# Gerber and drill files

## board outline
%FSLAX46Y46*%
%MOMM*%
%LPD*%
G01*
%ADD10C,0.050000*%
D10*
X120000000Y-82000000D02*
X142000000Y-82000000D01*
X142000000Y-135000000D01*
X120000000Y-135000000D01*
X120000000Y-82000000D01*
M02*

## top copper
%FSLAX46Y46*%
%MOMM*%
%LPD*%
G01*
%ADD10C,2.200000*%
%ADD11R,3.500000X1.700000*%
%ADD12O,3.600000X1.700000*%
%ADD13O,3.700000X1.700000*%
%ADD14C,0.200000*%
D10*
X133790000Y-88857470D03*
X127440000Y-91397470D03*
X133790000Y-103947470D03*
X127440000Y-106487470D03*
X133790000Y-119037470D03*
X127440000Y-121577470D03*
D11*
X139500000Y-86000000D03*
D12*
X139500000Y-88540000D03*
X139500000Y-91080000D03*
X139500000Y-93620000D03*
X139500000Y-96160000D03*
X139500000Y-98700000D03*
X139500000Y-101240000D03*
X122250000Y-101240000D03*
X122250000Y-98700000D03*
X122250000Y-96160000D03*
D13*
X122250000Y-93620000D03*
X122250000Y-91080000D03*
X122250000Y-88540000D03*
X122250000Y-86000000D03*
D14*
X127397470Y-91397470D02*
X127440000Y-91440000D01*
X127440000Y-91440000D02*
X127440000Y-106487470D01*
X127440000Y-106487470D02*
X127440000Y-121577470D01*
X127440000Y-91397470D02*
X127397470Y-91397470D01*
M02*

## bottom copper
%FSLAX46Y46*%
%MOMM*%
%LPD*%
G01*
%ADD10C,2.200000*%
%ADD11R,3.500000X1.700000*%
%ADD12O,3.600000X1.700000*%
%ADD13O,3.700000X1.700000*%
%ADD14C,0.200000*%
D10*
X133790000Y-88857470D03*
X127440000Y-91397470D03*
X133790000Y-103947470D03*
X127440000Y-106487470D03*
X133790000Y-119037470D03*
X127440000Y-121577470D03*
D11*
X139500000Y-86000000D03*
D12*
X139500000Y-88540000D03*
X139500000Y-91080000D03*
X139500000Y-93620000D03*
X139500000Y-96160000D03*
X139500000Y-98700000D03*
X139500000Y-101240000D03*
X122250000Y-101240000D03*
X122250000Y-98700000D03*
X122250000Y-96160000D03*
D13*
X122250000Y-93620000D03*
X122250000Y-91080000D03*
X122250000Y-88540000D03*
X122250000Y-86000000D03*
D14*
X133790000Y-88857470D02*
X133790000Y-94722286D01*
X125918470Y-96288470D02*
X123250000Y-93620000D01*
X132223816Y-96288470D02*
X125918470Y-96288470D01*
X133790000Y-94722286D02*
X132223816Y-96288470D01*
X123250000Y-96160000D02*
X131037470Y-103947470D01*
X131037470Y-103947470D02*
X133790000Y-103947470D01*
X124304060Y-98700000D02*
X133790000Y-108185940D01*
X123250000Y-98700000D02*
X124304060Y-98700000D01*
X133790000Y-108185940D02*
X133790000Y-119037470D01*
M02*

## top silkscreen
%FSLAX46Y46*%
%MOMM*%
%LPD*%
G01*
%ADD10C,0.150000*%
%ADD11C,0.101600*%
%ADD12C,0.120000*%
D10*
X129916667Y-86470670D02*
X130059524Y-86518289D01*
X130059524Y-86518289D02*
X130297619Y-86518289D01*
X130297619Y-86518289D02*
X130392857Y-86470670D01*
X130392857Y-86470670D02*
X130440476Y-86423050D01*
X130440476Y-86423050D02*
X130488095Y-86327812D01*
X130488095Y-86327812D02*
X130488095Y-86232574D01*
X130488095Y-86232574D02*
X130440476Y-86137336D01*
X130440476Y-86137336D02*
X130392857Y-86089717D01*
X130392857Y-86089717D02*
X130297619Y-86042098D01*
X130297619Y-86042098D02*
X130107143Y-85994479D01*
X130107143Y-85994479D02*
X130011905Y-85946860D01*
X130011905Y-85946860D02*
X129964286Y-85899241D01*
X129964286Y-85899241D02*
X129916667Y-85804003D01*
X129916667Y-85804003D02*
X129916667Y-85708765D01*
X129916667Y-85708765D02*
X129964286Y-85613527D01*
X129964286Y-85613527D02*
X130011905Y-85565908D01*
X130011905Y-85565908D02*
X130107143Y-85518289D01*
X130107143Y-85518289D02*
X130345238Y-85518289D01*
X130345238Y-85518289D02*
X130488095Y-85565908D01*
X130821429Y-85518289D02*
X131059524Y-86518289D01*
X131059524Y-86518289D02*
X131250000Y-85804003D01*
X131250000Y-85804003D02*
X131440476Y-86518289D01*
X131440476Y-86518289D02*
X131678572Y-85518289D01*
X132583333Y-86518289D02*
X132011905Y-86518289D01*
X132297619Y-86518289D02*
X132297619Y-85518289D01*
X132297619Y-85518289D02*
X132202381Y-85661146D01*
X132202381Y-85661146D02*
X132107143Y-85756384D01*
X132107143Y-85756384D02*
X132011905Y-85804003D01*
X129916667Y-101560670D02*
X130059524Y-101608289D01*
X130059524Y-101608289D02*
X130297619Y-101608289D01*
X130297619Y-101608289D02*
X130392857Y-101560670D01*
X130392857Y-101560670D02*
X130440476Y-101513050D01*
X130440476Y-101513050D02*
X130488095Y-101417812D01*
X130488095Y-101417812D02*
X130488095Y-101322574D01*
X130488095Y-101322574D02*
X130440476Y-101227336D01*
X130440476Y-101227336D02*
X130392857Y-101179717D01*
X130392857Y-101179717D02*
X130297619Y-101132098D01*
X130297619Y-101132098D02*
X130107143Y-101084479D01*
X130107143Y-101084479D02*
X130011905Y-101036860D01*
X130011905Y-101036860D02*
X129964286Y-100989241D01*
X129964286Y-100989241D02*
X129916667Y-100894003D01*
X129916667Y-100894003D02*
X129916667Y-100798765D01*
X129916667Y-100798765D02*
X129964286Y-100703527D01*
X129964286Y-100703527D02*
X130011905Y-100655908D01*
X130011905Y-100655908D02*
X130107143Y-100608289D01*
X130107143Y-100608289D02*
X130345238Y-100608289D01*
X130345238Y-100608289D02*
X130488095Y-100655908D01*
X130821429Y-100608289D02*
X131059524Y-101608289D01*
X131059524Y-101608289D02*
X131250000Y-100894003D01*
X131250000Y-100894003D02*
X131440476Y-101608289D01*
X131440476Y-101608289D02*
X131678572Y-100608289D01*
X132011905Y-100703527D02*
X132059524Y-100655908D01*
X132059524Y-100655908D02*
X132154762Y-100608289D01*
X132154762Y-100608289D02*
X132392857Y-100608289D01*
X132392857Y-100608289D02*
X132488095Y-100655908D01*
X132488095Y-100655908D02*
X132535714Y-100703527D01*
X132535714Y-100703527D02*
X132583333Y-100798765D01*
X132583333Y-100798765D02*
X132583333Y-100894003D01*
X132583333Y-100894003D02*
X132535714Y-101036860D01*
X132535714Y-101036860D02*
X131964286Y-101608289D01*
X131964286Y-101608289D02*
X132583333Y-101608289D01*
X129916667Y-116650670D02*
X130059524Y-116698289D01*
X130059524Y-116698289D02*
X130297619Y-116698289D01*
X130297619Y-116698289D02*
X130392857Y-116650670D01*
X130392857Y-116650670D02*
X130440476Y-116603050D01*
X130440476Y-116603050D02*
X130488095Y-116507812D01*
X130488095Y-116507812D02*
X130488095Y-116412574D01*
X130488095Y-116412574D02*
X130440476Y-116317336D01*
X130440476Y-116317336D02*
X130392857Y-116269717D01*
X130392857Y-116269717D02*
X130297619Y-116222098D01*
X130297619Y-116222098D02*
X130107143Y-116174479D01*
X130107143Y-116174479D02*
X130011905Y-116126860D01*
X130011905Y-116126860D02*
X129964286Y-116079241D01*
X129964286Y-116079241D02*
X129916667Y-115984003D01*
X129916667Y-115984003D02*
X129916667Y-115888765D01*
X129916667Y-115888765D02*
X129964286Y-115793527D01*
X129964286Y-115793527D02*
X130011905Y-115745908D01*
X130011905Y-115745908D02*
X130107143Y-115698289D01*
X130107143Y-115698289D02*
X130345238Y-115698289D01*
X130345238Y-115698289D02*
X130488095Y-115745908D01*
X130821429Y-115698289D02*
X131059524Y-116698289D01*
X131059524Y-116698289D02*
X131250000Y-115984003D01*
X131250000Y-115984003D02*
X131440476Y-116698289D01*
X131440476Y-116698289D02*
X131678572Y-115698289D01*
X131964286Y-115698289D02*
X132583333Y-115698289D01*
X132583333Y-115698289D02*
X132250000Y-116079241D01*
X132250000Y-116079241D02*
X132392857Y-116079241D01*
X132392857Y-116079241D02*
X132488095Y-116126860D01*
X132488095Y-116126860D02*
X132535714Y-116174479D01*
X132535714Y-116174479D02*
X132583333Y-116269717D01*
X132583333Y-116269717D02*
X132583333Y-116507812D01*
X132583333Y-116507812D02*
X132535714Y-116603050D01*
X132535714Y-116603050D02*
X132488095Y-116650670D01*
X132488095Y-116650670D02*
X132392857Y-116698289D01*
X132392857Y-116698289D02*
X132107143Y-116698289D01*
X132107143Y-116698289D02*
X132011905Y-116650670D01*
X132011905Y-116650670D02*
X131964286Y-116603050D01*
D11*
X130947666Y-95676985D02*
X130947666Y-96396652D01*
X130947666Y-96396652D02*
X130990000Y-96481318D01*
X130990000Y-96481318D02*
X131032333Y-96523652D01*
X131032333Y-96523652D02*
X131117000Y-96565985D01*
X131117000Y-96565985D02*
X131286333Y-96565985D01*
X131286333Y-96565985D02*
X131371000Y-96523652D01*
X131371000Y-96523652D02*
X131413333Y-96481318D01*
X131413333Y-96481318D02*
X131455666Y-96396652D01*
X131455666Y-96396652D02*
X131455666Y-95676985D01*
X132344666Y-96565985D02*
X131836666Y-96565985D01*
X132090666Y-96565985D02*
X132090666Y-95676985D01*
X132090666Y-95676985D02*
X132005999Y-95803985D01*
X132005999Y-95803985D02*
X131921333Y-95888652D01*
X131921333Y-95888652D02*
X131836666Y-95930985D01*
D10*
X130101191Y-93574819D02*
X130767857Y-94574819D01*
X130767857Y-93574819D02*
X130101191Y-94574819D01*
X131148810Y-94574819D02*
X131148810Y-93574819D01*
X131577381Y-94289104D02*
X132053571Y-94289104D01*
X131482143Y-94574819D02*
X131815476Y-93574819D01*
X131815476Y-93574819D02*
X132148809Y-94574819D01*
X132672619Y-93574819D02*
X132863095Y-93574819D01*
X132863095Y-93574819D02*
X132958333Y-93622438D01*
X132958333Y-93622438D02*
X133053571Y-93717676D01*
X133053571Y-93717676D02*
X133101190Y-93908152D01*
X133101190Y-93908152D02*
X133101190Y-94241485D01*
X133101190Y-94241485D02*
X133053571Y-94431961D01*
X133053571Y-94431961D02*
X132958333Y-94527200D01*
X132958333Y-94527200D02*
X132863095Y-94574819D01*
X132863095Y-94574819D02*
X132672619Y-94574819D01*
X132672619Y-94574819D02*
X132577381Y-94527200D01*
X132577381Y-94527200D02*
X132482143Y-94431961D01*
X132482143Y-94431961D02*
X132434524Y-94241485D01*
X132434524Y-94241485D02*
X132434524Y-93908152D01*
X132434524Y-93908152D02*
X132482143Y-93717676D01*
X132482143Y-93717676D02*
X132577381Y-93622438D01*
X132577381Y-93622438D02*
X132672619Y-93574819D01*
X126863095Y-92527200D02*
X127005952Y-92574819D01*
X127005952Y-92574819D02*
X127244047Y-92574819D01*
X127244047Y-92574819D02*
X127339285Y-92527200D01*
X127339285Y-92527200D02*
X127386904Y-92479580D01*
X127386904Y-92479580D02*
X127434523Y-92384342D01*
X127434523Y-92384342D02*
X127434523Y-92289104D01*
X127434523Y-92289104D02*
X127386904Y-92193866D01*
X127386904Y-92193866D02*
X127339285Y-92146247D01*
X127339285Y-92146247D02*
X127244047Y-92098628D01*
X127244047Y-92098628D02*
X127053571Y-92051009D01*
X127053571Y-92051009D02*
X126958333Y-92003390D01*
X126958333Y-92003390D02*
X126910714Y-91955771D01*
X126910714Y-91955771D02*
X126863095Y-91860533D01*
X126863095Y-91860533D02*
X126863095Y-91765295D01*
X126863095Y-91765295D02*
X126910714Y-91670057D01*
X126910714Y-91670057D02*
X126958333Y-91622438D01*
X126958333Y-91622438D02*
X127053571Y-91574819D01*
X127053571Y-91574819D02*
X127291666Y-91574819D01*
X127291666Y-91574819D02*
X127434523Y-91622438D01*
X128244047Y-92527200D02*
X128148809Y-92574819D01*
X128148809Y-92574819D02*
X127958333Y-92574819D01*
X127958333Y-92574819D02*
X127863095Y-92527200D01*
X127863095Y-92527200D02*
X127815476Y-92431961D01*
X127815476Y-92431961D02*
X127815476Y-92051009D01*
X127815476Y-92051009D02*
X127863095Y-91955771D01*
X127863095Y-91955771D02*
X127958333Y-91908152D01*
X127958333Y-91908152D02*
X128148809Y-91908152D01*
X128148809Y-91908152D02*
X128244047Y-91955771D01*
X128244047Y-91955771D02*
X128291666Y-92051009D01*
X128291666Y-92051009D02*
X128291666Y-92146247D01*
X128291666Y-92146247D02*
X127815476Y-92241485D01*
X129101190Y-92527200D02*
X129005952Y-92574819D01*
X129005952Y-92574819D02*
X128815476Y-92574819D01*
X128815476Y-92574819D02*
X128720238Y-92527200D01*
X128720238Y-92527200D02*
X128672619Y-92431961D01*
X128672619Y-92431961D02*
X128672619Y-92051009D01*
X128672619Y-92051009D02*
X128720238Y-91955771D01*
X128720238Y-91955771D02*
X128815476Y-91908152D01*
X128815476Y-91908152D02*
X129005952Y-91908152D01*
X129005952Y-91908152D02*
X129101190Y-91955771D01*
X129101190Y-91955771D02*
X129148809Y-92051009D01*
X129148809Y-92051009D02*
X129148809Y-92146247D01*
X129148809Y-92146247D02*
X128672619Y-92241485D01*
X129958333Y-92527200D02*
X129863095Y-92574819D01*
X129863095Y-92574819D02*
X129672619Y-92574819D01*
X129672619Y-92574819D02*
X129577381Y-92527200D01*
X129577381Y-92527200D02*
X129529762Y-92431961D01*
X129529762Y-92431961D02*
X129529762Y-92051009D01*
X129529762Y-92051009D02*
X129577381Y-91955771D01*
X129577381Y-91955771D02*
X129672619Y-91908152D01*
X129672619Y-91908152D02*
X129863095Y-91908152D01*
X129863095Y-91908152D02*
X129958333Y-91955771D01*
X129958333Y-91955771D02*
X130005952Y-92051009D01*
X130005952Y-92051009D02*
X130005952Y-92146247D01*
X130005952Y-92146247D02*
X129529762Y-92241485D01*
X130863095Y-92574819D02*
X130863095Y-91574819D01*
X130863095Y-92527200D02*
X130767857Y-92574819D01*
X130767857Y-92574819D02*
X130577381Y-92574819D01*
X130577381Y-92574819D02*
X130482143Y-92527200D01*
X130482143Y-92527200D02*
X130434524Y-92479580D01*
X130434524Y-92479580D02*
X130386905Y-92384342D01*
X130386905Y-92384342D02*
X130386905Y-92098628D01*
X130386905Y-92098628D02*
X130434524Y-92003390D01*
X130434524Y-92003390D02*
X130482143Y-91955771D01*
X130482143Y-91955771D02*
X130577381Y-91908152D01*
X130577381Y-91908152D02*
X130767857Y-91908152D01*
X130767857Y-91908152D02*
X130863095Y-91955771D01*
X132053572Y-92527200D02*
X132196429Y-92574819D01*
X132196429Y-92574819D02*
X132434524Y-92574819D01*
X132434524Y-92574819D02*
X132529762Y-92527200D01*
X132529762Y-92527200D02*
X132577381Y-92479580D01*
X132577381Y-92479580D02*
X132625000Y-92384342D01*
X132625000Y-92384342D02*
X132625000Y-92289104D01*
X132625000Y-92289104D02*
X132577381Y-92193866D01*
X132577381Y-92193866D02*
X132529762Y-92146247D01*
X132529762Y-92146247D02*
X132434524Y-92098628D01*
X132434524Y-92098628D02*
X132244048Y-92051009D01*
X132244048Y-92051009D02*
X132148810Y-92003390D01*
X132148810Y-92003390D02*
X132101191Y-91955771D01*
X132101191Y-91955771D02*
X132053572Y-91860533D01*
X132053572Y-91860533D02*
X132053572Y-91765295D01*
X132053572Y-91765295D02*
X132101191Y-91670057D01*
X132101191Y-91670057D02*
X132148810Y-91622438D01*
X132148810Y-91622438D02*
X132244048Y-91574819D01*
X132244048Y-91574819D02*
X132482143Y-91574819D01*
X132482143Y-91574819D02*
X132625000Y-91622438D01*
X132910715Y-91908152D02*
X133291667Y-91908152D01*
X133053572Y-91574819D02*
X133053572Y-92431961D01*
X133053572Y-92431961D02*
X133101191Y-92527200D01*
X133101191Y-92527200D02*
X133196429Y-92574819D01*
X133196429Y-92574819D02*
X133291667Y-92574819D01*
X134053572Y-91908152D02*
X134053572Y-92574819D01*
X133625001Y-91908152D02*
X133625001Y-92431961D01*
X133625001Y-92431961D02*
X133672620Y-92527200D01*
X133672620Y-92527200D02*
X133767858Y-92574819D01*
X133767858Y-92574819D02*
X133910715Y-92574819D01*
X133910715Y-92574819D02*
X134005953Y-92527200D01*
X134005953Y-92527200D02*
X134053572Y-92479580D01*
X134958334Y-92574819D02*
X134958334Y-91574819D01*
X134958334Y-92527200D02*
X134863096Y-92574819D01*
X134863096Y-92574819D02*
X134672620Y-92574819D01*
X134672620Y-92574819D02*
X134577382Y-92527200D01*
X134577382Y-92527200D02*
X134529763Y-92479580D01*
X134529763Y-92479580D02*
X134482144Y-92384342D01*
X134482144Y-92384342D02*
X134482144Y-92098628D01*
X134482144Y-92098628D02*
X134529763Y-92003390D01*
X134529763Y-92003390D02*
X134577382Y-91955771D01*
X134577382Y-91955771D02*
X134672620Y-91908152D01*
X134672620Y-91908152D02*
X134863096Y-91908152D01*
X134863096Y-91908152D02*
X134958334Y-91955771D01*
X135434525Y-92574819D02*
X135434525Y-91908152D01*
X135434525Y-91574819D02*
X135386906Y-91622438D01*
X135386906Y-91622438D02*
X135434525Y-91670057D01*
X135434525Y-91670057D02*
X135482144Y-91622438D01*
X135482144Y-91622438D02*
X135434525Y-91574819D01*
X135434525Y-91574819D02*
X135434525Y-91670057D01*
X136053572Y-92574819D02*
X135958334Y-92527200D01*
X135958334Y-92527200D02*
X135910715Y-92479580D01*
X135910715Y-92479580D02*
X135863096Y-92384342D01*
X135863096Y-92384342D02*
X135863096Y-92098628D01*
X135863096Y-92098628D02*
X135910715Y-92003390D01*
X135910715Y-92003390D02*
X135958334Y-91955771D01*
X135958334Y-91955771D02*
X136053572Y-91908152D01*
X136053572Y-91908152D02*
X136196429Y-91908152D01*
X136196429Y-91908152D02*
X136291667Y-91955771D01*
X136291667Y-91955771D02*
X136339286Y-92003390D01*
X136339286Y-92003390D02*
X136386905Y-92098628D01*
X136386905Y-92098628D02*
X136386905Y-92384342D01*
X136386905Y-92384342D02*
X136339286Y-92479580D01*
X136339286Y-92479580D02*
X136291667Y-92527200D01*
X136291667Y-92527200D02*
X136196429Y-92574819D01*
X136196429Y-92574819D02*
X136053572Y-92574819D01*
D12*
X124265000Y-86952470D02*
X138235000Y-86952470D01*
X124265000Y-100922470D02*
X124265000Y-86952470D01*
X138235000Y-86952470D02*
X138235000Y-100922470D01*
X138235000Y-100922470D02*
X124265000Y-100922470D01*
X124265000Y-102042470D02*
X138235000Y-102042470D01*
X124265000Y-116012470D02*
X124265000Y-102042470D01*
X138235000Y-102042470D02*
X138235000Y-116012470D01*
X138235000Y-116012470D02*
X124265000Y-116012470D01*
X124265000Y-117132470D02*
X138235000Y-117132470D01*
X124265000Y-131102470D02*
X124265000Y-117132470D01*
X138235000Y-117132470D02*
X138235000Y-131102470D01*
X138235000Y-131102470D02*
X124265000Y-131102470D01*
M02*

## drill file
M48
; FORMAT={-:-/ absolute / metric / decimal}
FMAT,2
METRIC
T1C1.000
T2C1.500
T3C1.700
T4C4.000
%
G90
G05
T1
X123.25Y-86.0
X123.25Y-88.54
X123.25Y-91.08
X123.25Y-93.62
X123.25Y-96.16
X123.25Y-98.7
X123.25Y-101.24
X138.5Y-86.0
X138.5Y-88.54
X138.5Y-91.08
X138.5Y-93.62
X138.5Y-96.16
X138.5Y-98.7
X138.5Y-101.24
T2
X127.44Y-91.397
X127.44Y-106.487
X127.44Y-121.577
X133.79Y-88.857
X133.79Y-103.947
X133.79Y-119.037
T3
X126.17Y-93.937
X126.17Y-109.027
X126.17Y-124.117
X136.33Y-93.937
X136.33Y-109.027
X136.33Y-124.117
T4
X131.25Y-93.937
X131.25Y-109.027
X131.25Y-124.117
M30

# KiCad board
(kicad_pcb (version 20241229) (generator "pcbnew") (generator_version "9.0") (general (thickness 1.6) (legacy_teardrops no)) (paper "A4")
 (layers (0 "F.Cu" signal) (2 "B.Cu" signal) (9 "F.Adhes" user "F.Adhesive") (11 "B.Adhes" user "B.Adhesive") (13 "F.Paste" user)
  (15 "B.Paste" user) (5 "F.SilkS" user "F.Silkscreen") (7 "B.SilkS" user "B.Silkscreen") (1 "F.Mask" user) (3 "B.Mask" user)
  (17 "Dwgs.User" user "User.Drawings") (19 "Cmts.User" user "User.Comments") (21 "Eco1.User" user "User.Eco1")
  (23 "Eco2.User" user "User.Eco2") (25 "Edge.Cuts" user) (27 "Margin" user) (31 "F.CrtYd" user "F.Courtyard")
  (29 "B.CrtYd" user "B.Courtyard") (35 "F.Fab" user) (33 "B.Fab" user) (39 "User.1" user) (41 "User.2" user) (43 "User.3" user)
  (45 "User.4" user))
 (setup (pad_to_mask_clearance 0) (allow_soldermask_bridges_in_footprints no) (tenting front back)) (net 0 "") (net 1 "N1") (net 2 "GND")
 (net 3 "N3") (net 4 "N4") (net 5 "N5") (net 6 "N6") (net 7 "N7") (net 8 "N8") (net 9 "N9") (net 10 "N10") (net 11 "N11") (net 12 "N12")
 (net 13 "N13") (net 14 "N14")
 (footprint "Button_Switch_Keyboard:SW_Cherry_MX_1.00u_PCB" (layer "F.Cu") (at 133.79 88.85747)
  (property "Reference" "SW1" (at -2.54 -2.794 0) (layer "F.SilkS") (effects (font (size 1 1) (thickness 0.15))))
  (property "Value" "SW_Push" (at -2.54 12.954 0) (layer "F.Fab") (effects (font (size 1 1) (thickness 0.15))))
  (fp_line (start -9.525 -1.905) (end 4.445 -1.905) (stroke (width 0.12) (type solid)) (layer "F.SilkS"))
  (fp_line (start -9.525 12.065) (end -9.525 -1.905) (stroke (width 0.12) (type solid)) (layer "F.SilkS"))
  (fp_line (start 4.445 -1.905) (end 4.445 12.065) (stroke (width 0.12) (type solid)) (layer "F.SilkS"))
  (fp_line (start 4.445 12.065) (end -9.525 12.065) (stroke (width 0.12) (type solid)) (layer "F.SilkS"))
  (pad "" np_thru_hole circle (at -7.62 5.08) (size 1.7 1.7) (drill 1.7) (layers "*.Cu" "*.Mask"))
  (pad "" np_thru_hole circle (at -2.54 5.08) (size 4 4) (drill 4) (layers "*.Cu" "*.Mask"))
  (pad "" np_thru_hole circle (at 2.54 5.08) (size 1.7 1.7) (drill 1.7) (layers "*.Cu" "*.Mask"))
  (pad "1" thru_hole circle (at 0 0) (size 2.2 2.2) (drill 1.5) (layers "*.Cu" "*.Mask") (remove_unused_layers no) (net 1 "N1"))
  (pad "2" thru_hole circle (at -6.35 2.54) (size 2.2 2.2) (drill 1.5) (layers "*.Cu" "*.Mask") (remove_unused_layers no) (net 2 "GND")))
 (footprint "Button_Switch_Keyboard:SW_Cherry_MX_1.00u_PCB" (layer "F.Cu") (at 133.79 103.94747)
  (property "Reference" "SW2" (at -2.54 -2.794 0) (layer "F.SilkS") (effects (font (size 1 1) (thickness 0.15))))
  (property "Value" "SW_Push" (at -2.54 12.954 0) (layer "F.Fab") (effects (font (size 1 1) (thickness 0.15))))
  (fp_line (start -9.525 -1.905) (end 4.445 -1.905) (stroke (width 0.12) (type solid)) (layer "F.SilkS"))
  (fp_line (start -9.525 12.065) (end -9.525 -1.905) (stroke (width 0.12) (type solid)) (layer "F.SilkS"))
  (fp_line (start 4.445 -1.905) (end 4.445 12.065) (stroke (width 0.12) (type solid)) (layer "F.SilkS"))
  (fp_line (start 4.445 12.065) (end -9.525 12.065) (stroke (width 0.12) (type solid)) (layer "F.SilkS"))
  (pad "" np_thru_hole circle (at -7.62 5.08) (size 1.7 1.7) (drill 1.7) (layers "*.Cu" "*.Mask"))
  (pad "" np_thru_hole circle (at -2.54 5.08) (size 4 4) (drill 4) (layers "*.Cu" "*.Mask"))
  (pad "" np_thru_hole circle (at 2.54 5.08) (size 1.7 1.7) (drill 1.7) (layers "*.Cu" "*.Mask"))
  (pad "1" thru_hole circle (at 0 0) (size 2.2 2.2) (drill 1.5) (layers "*.Cu" "*.Mask") (remove_unused_layers no) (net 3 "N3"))
  (pad "2" thru_hole circle (at -6.35 2.54) (size 2.2 2.2) (drill 1.5) (layers "*.Cu" "*.Mask") (remove_unused_layers no) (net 2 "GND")))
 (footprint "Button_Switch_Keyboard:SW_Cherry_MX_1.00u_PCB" (layer "F.Cu") (at 133.79 119.03747)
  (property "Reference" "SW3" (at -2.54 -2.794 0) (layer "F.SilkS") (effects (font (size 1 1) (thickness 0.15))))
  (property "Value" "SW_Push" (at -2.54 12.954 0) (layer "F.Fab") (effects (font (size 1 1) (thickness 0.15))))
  (fp_line (start -9.525 -1.905) (end 4.445 -1.905) (stroke (width 0.12) (type solid)) (layer "F.SilkS"))
  (fp_line (start -9.525 12.065) (end -9.525 -1.905) (stroke (width 0.12) (type solid)) (layer "F.SilkS"))
  (fp_line (start 4.445 -1.905) (end 4.445 12.065) (stroke (width 0.12) (type solid)) (layer "F.SilkS"))
  (fp_line (start 4.445 12.065) (end -9.525 12.065) (stroke (width 0.12) (type solid)) (layer "F.SilkS"))
  (pad "" np_thru_hole circle (at -7.62 5.08) (size 1.7 1.7) (drill 1.7) (layers "*.Cu" "*.Mask"))
  (pad "" np_thru_hole circle (at -2.54 5.08) (size 4 4) (drill 4) (layers "*.Cu" "*.Mask"))
  (pad "" np_thru_hole circle (at 2.54 5.08) (size 1.7 1.7) (drill 1.7) (layers "*.Cu" "*.Mask"))
  (pad "1" thru_hole circle (at 0 0) (size 2.2 2.2) (drill 1.5) (layers "*.Cu" "*.Mask") (remove_unused_layers no) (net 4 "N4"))
  (pad "2" thru_hole circle (at -6.35 2.54) (size 2.2 2.2) (drill 1.5) (layers "*.Cu" "*.Mask") (remove_unused_layers no) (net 2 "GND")))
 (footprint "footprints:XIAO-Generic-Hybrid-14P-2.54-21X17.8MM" (layer "B.Cu") (at 130.875 93.62 180)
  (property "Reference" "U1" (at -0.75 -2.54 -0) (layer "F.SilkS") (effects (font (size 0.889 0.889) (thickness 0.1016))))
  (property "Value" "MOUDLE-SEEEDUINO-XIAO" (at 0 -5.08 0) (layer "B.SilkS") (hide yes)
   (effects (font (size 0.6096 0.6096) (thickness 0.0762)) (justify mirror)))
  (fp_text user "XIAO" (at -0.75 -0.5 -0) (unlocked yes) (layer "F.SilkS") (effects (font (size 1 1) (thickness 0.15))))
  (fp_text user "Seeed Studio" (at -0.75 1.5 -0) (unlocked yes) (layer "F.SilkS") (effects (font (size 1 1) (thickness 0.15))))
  (pad "1" thru_hole rect (at -7.625 7.62 180) (size 3.5 1.7) (drill 1 (offset -1 0)) (layers "*.Cu" "*.Mask") (remove_unused_layers no)
   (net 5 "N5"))
  (pad "2" thru_hole oval (at -7.625 5.08 180) (size 3.6 1.7) (drill 1 (offset -1 0)) (layers "*.Cu" "*.Mask") (remove_unused_layers no)
   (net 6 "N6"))
  (pad "3" thru_hole oval (at -7.625 2.54 180) (size 3.6 1.7) (drill 1 (offset -1 0)) (layers "*.Cu" "*.Mask") (remove_unused_layers no)
   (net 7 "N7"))
  (pad "4" thru_hole oval (at -7.625 0 180) (size 3.6 1.7) (drill 1 (offset -1 0)) (layers "*.Cu" "*.Mask") (remove_unused_layers no)
   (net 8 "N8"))
  (pad "5" thru_hole oval (at -7.625 -2.54 180) (size 3.6 1.7) (drill 1 (offset -1 0)) (layers "*.Cu" "*.Mask") (remove_unused_layers no)
   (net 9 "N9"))
  (pad "6" thru_hole oval (at -7.625 -5.08) (size 3.6 1.7) (drill 1 (offset 1 0)) (layers "*.Cu" "*.Mask") (remove_unused_layers no)
   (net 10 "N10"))
  (pad "7" thru_hole oval (at -7.625 -7.62 180) (size 3.6 1.7) (drill 1 (offset -1 0)) (layers "*.Cu" "*.Mask") (remove_unused_layers no)
   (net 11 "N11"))
  (pad "8" thru_hole oval (at 7.625 -7.62 180) (size 3.6 1.7) (drill 1 (offset 1 0)) (layers "*.Cu" "*.Mask") (remove_unused_layers no)
   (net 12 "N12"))
  (pad "9" thru_hole oval (at 7.625 -5.08 180) (size 3.6 1.7) (drill 1 (offset 1 0)) (layers "*.Cu" "*.Mask") (remove_unused_layers no)
   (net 4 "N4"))
  (pad "10" thru_hole oval (at 7.625 -2.54 180) (size 3.6 1.7) (drill 1 (offset 1 0)) (layers "*.Cu" "*.Mask") (remove_unused_layers no)
   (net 3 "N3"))
  (pad "11" thru_hole oval (at 7.625 0 180) (size 3.7 1.7) (drill 1 (offset 1 0)) (layers "*.Cu" "*.Mask") (remove_unused_layers no)
   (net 1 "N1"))
  (pad "12" thru_hole oval (at 7.625 2.54 180) (size 3.7 1.7) (drill 1 (offset 1 0)) (layers "*.Cu" "*.Mask") (remove_unused_layers no)
   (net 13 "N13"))
  (pad "13" thru_hole oval (at 7.625 5.08 180) (size 3.7 1.7) (drill 1 (offset 1 0)) (layers "*.Cu" "*.Mask") (remove_unused_layers no)
   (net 2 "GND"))
  (pad "14" thru_hole oval (at 7.625 7.62 180) (size 3.7 1.7) (drill 1 (offset 1 0)) (layers "*.Cu" "*.Mask") (remove_unused_layers no)
   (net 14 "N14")))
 (gr_rect (start 120 82) (end 142 135) (stroke (width 0.05) (type default)) (fill no) (layer "Edge.Cuts"))
 (segment (start 133.79 88.85747) (end 133.79 94.722286) (width 0.2) (layer "B.Cu") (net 1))
 (segment (start 125.91847 96.28847) (end 123.25 93.62) (width 0.2) (layer "B.Cu") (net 1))
 (segment (start 132.223816 96.28847) (end 125.91847 96.28847) (width 0.2) (layer "B.Cu") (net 1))
 (segment (start 133.79 94.722286) (end 132.223816 96.28847) (width 0.2) (layer "B.Cu") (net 1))
 (segment (start 127.39747 91.39747) (end 127.44 91.44) (width 0.2) (layer "F.Cu") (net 2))
 (segment (start 127.44 91.44) (end 127.44 106.48747) (width 0.2) (layer "F.Cu") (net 2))
 (segment (start 127.44 106.48747) (end 127.44 121.57747) (width 0.2) (layer "F.Cu") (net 2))
 (segment (start 127.44 91.39747) (end 127.39747 91.39747) (width 0.2) (layer "F.Cu") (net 2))
 (segment (start 123.25 96.16) (end 131.03747 103.94747) (width 0.2) (layer "B.Cu") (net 3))
 (segment (start 131.03747 103.94747) (end 133.79 103.94747) (width 0.2) (layer "B.Cu") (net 3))
 (segment (start 124.30406 98.7) (end 133.79 108.18594) (width 0.2) (layer "B.Cu") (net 4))
 (segment (start 123.25 98.7) (end 124.30406 98.7) (width 0.2) (layer "B.Cu") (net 4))
 (segment (start 133.79 108.18594) (end 133.79 119.03747) (width 0.2) (layer "B.Cu") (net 4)))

